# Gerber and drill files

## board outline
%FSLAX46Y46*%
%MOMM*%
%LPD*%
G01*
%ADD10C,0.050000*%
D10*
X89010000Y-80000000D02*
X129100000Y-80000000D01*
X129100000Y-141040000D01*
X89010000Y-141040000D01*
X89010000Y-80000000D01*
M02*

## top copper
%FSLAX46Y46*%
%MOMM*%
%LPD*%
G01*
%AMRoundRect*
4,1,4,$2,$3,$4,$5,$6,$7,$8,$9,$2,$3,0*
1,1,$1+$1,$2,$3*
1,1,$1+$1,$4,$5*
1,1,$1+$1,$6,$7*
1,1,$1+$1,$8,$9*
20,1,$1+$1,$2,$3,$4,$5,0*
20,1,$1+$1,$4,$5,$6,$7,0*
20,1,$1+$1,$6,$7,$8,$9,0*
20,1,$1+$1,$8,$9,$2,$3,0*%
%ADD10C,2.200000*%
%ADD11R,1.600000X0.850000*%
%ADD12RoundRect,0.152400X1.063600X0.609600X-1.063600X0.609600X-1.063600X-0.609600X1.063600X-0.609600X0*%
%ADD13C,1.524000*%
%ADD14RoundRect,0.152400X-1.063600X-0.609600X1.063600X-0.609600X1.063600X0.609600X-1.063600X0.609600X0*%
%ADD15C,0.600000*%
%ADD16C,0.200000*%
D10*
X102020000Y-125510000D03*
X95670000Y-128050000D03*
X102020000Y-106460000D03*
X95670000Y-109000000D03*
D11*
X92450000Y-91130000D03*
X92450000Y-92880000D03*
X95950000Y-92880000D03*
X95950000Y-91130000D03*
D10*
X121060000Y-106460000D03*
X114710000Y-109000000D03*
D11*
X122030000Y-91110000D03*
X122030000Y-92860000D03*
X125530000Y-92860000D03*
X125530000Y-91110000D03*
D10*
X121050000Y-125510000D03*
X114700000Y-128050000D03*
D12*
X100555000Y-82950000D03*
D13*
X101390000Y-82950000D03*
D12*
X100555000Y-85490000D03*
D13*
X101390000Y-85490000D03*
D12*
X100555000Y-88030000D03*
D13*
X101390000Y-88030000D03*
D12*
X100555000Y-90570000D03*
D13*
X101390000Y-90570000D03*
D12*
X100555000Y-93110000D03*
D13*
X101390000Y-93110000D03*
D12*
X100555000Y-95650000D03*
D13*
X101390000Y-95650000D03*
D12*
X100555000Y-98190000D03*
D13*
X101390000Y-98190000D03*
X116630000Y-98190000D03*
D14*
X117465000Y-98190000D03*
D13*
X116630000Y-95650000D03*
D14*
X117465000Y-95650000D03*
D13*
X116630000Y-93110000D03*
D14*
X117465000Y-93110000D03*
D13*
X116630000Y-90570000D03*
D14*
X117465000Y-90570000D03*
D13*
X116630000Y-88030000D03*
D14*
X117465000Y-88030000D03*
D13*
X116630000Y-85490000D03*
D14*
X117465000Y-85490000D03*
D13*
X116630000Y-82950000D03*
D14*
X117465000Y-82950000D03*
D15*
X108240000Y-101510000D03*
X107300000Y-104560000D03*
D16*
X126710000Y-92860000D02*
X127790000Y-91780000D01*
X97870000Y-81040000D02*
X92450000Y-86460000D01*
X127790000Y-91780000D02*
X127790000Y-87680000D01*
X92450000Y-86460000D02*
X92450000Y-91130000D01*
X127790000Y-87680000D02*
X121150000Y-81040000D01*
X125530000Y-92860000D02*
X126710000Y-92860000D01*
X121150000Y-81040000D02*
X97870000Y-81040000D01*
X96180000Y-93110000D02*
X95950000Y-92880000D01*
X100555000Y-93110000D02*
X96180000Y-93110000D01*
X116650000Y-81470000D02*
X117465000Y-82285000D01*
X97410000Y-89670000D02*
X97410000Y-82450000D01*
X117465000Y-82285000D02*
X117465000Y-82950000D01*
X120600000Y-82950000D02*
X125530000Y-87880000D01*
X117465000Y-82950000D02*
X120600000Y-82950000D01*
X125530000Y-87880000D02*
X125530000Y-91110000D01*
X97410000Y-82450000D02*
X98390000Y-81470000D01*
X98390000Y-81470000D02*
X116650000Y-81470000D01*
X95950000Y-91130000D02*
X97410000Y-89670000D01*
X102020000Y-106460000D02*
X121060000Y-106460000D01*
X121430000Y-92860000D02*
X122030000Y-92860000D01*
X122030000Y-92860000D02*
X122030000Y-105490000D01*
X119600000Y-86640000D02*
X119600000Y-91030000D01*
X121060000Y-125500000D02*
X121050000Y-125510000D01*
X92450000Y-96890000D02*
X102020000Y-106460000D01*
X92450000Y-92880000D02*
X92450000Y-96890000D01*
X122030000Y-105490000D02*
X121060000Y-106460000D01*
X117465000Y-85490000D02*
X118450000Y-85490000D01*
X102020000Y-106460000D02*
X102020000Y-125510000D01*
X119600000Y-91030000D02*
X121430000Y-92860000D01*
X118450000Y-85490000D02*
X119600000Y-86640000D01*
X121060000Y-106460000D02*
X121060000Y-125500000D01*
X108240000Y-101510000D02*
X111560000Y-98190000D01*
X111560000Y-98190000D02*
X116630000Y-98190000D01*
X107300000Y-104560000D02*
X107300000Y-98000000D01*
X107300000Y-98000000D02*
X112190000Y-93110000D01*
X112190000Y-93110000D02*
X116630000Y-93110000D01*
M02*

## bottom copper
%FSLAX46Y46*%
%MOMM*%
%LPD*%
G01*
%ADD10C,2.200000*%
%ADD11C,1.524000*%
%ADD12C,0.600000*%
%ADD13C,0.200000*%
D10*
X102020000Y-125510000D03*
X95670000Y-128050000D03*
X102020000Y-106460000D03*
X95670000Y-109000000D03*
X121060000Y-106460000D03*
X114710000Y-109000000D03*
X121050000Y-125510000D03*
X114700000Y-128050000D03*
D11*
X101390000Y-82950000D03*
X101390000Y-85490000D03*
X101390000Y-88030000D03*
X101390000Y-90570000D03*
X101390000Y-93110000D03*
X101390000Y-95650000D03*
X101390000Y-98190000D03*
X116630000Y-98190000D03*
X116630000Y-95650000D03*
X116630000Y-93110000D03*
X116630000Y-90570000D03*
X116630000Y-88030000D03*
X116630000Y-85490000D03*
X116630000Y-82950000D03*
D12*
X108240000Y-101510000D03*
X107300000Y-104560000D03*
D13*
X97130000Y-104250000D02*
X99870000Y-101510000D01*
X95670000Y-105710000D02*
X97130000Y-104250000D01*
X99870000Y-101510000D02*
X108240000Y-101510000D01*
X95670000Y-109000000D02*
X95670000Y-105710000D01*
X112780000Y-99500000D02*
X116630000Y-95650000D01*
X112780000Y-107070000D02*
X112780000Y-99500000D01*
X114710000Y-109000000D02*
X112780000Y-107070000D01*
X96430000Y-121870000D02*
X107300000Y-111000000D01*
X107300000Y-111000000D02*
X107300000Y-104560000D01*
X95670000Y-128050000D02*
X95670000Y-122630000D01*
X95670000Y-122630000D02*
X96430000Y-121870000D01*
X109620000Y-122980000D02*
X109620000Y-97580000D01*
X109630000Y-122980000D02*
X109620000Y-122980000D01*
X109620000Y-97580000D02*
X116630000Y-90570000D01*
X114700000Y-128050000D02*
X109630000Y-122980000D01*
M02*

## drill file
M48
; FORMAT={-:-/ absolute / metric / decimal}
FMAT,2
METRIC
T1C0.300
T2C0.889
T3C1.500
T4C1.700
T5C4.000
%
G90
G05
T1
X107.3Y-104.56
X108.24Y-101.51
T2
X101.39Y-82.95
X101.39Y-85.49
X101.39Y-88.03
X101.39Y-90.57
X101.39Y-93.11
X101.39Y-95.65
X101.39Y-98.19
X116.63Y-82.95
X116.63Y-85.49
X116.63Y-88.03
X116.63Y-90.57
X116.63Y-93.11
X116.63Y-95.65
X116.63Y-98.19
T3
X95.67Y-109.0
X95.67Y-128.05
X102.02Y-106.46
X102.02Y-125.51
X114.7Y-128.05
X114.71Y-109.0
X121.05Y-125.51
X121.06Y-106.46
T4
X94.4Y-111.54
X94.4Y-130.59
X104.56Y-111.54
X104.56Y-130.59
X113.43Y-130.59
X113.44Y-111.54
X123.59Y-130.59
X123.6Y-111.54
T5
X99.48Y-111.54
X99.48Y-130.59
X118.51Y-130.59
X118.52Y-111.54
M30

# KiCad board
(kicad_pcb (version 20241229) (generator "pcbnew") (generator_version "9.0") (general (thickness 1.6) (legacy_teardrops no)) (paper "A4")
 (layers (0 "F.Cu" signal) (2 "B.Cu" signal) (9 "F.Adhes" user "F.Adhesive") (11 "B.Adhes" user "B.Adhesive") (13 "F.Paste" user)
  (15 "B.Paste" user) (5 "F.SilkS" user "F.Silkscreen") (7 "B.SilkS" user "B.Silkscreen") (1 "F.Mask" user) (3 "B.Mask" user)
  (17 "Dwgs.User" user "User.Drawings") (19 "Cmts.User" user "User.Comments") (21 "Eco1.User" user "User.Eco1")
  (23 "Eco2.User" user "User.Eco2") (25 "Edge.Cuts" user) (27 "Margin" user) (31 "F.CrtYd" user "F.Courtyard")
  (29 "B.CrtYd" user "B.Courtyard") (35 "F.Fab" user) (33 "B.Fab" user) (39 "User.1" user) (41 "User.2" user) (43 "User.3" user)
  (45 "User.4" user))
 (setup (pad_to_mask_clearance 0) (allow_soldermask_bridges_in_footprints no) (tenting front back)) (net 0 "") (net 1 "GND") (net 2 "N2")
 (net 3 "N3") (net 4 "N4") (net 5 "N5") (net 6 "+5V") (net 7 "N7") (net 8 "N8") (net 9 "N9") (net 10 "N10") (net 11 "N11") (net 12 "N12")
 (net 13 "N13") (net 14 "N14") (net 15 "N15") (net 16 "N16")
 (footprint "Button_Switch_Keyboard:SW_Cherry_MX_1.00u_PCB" (layer "F.Cu") (at 102.02 125.51)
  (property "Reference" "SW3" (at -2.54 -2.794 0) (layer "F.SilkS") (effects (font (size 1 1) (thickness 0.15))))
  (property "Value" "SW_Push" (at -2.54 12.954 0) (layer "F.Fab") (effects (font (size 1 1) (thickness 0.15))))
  (pad "" np_thru_hole circle (at -7.62 5.08) (size 1.7 1.7) (drill 1.7) (layers "*.Cu" "*.Mask"))
  (pad "" np_thru_hole circle (at -2.54 5.08) (size 4 4) (drill 4) (layers "*.Cu" "*.Mask"))
  (pad "" np_thru_hole circle (at 2.54 5.08) (size 1.7 1.7) (drill 1.7) (layers "*.Cu" "*.Mask"))
  (pad "1" thru_hole circle (at 0 0) (size 2.2 2.2) (drill 1.5) (layers "*.Cu" "*.Mask") (remove_unused_layers no) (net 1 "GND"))
  (pad "2" thru_hole circle (at -6.35 2.54) (size 2.2 2.2) (drill 1.5) (layers "*.Cu" "*.Mask") (remove_unused_layers no) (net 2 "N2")))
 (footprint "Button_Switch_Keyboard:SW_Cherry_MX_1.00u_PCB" (layer "F.Cu") (at 102.02 106.46)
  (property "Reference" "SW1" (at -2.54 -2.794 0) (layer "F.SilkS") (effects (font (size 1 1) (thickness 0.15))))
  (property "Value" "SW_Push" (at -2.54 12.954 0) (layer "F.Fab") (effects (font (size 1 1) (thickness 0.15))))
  (pad "" np_thru_hole circle (at -7.62 5.08) (size 1.7 1.7) (drill 1.7) (layers "*.Cu" "*.Mask"))
  (pad "" np_thru_hole circle (at -2.54 5.08) (size 4 4) (drill 4) (layers "*.Cu" "*.Mask"))
  (pad "" np_thru_hole circle (at 2.54 5.08) (size 1.7 1.7) (drill 1.7) (layers "*.Cu" "*.Mask"))
  (pad "1" thru_hole circle (at 0 0) (size 2.2 2.2) (drill 1.5) (layers "*.Cu" "*.Mask") (remove_unused_layers no) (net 1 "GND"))
  (pad "2" thru_hole circle (at -6.35 2.54) (size 2.2 2.2) (drill 1.5) (layers "*.Cu" "*.Mask") (remove_unused_layers no) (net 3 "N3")))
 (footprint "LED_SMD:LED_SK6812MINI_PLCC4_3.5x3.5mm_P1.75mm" (layer "F.Cu") (at 94.2 92.005)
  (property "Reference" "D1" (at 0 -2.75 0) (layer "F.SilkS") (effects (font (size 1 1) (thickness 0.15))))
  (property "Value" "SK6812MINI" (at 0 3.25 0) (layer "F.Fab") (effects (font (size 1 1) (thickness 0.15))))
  (pad "1" smd rect (at -1.75 -0.875) (size 1.6 0.85) (layers "F.Cu" "F.Mask" "F.Paste") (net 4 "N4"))
  (pad "2" smd rect (at -1.75 0.875) (size 1.6 0.85) (layers "F.Cu" "F.Mask" "F.Paste") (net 1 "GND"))
  (pad "3" smd rect (at 1.75 0.875) (size 1.6 0.85) (layers "F.Cu" "F.Mask" "F.Paste") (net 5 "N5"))
  (pad "4" smd rect (at 1.75 -0.875) (size 1.6 0.85) (layers "F.Cu" "F.Mask" "F.Paste") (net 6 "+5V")))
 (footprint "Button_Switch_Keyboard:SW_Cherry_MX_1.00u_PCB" (layer "F.Cu") (at 121.06 106.46)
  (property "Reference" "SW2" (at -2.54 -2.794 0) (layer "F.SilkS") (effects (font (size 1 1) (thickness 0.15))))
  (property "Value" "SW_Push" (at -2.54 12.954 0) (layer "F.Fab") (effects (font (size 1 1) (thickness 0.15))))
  (pad "" np_thru_hole circle (at -7.62 5.08) (size 1.7 1.7) (drill 1.7) (layers "*.Cu" "*.Mask"))
  (pad "" np_thru_hole circle (at -2.54 5.08) (size 4 4) (drill 4) (layers "*.Cu" "*.Mask"))
  (pad "" np_thru_hole circle (at 2.54 5.08) (size 1.7 1.7) (drill 1.7) (layers "*.Cu" "*.Mask"))
  (pad "1" thru_hole circle (at 0 0) (size 2.2 2.2) (drill 1.5) (layers "*.Cu" "*.Mask") (remove_unused_layers no) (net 1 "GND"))
  (pad "2" thru_hole circle (at -6.35 2.54) (size 2.2 2.2) (drill 1.5) (layers "*.Cu" "*.Mask") (remove_unused_layers no) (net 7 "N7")))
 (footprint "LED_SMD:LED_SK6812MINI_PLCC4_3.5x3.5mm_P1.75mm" (layer "F.Cu") (at 123.78 91.985)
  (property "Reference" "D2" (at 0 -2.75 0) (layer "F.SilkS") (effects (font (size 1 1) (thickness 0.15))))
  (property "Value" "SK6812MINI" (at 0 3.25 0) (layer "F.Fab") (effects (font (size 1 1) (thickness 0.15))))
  (pad "1" smd rect (at -1.75 -0.875) (size 1.6 0.85) (layers "F.Cu" "F.Mask" "F.Paste") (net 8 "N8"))
  (pad "2" smd rect (at -1.75 0.875) (size 1.6 0.85) (layers "F.Cu" "F.Mask" "F.Paste") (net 1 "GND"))
  (pad "3" smd rect (at 1.75 0.875) (size 1.6 0.85) (layers "F.Cu" "F.Mask" "F.Paste") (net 4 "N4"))
  (pad "4" smd rect (at 1.75 -0.875) (size 1.6 0.85) (layers "F.Cu" "F.Mask" "F.Paste") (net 6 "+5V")))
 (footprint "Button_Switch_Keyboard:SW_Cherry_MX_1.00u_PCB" (layer "F.Cu") (at 121.05 125.51)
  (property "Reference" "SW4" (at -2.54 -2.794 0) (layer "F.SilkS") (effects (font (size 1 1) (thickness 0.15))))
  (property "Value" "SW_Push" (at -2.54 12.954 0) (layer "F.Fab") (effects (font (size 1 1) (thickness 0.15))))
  (pad "" np_thru_hole circle (at -7.62 5.08) (size 1.7 1.7) (drill 1.7) (layers "*.Cu" "*.Mask"))
  (pad "" np_thru_hole circle (at -2.54 5.08) (size 4 4) (drill 4) (layers "*.Cu" "*.Mask"))
  (pad "" np_thru_hole circle (at 2.54 5.08) (size 1.7 1.7) (drill 1.7) (layers "*.Cu" "*.Mask"))
  (pad "1" thru_hole circle (at 0 0) (size 2.2 2.2) (drill 1.5) (layers "*.Cu" "*.Mask") (remove_unused_layers no) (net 1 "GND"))
  (pad "2" thru_hole circle (at -6.35 2.54) (size 2.2 2.2) (drill 1.5) (layers "*.Cu" "*.Mask") (remove_unused_layers no) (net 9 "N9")))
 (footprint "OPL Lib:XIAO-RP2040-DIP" (layer "F.Cu") (at 109.01 90.57)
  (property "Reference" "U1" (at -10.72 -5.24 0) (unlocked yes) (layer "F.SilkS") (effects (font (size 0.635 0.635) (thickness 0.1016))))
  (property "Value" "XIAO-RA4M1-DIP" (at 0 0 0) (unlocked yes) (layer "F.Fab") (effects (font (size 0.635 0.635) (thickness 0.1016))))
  (pad "1" smd roundrect (at -8.455 -7.62 180) (size 2.432 1.524) (layers "F.Cu" "F.Mask") (roundrect_rratio 0.1) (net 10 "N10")
   (thermal_bridge_angle 45))
  (pad "1" thru_hole circle (at -7.62 -7.62 180) (size 1.524 1.524) (drill 0.889) (layers "*.Cu" "*.Mask") (remove_unused_layers no)
   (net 10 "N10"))
  (pad "2" smd roundrect (at -8.455 -5.08 180) (size 2.432 1.524) (layers "F.Cu" "F.Mask") (roundrect_rratio 0.1) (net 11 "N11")
   (thermal_bridge_angle 45))
  (pad "2" thru_hole circle (at -7.62 -5.08 180) (size 1.524 1.524) (drill 0.889) (layers "*.Cu" "*.Mask") (remove_unused_layers no)
   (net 11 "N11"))
  (pad "3" smd roundrect (at -8.455 -2.54 180) (size 2.432 1.524) (layers "F.Cu" "F.Mask") (roundrect_rratio 0.1) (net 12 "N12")
   (thermal_bridge_angle 45))
  (pad "3" thru_hole circle (at -7.62 -2.54 180) (size 1.524 1.524) (drill 0.889) (layers "*.Cu" "*.Mask") (remove_unused_layers no)
   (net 12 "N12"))
  (pad "4" smd roundrect (at -8.455 0 180) (size 2.432 1.524) (layers "F.Cu" "F.Mask") (roundrect_rratio 0.1) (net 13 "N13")
   (thermal_bridge_angle 45))
  (pad "4" thru_hole circle (at -7.62 0 180) (size 1.524 1.524) (drill 0.889) (layers "*.Cu" "*.Mask") (remove_unused_layers no)
   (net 13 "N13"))
  (pad "5" smd roundrect (at -8.455 2.54 180) (size 2.432 1.524) (layers "F.Cu" "F.Mask") (roundrect_rratio 0.1) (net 5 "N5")
   (thermal_bridge_angle 45))
  (pad "5" thru_hole circle (at -7.62 2.54 180) (size 1.524 1.524) (drill 0.889) (layers "*.Cu" "*.Mask") (remove_unused_layers no)
   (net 5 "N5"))
  (pad "6" smd roundrect (at -8.455 5.08 180) (size 2.432 1.524) (layers "F.Cu" "F.Mask") (roundrect_rratio 0.1) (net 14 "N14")
   (thermal_bridge_angle 45))
  (pad "6" thru_hole circle (at -7.62 5.08 180) (size 1.524 1.524) (drill 0.889) (layers "*.Cu" "*.Mask") (remove_unused_layers no)
   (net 14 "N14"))
  (pad "7" smd roundrect (at -8.455 7.62 180) (size 2.432 1.524) (layers "F.Cu" "F.Mask") (roundrect_rratio 0.1) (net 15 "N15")
   (thermal_bridge_angle 45))
  (pad "7" thru_hole circle (at -7.62 7.62 180) (size 1.524 1.524) (drill 0.889) (layers "*.Cu" "*.Mask") (remove_unused_layers no)
   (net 15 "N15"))
  (pad "8" thru_hole circle (at 7.62 7.62) (size 1.524 1.524) (drill 0.889) (layers "*.Cu" "*.Mask") (remove_unused_layers no) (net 3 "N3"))
  (pad "8" smd roundrect (at 8.455 7.62) (size 2.432 1.524) (layers "F.Cu" "F.Mask") (roundrect_rratio 0.1) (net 3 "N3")
   (thermal_bridge_angle 45))
  (pad "9" thru_hole circle (at 7.62 5.08) (size 1.524 1.524) (drill 0.889) (layers "*.Cu" "*.Mask") (remove_unused_layers no) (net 7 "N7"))
  (pad "9" smd roundrect (at 8.455 5.08) (size 2.432 1.524) (layers "F.Cu" "F.Mask") (roundrect_rratio 0.1) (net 7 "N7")
   (thermal_bridge_angle 45))
  (pad "10" thru_hole circle (at 7.62 2.54) (size 1.524 1.524) (drill 0.889) (layers "*.Cu" "*.Mask") (remove_unused_layers no) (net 2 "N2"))
  (pad "10" smd roundrect (at 8.455 2.54) (size 2.432 1.524) (layers "F.Cu" "F.Mask") (roundrect_rratio 0.1) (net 2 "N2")
   (thermal_bridge_angle 45))
  (pad "11" thru_hole circle (at 7.62 0) (size 1.524 1.524) (drill 0.889) (layers "*.Cu" "*.Mask") (remove_unused_layers no) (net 9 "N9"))
  (pad "11" smd roundrect (at 8.455 0) (size 2.432 1.524) (layers "F.Cu" "F.Mask") (roundrect_rratio 0.1) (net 9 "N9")
   (thermal_bridge_angle 45))
  (pad "12" thru_hole circle (at 7.62 -2.54) (size 1.524 1.524) (drill 0.889) (layers "*.Cu" "*.Mask") (remove_unused_layers no)
   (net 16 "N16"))
  (pad "12" smd roundrect (at 8.455 -2.54) (size 2.432 1.524) (layers "F.Cu" "F.Mask") (roundrect_rratio 0.1) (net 16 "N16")
   (thermal_bridge_angle 45))
  (pad "13" thru_hole circle (at 7.62 -5.08) (size 1.524 1.524) (drill 0.889) (layers "*.Cu" "*.Mask") (remove_unused_layers no)
   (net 1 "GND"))
  (pad "13" smd roundrect (at 8.455 -5.08) (size 2.432 1.524) (layers "F.Cu" "F.Mask") (roundrect_rratio 0.1) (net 1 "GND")
   (thermal_bridge_angle 45))
  (pad "14" thru_hole circle (at 7.62 -7.62) (size 1.524 1.524) (drill 0.889) (layers "*.Cu" "*.Mask") (remove_unused_layers no)
   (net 6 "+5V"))
  (pad "14" smd roundrect (at 8.455 -7.62) (size 2.432 1.524) (layers "F.Cu" "F.Mask") (roundrect_rratio 0.1) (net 6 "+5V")
   (thermal_bridge_angle 45)))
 (gr_rect (start 89.01 80) (end 129.1 141.04) (stroke (width 0.05) (type default)) (fill no) (layer "Edge.Cuts"))
 (segment (start 126.71 92.86) (end 127.79 91.78) (width 0.2) (layer "F.Cu") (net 4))
 (segment (start 97.87 81.04) (end 92.45 86.46) (width 0.2) (layer "F.Cu") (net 4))
 (segment (start 127.79 91.78) (end 127.79 87.68) (width 0.2) (layer "F.Cu") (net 4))
 (segment (start 92.45 86.46) (end 92.45 91.13) (width 0.2) (layer "F.Cu") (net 4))
 (segment (start 127.79 87.68) (end 121.15 81.04) (width 0.2) (layer "F.Cu") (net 4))
 (segment (start 125.53 92.86) (end 126.71 92.86) (width 0.2) (layer "F.Cu") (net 4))
 (segment (start 121.15 81.04) (end 97.87 81.04) (width 0.2) (layer "F.Cu") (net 4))
 (segment (start 96.18 93.11) (end 95.95 92.88) (width 0.2) (layer "F.Cu") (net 5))
 (segment (start 100.555 93.11) (end 96.18 93.11) (width 0.2) (layer "F.Cu") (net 5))
 (segment (start 116.65 81.47) (end 117.465 82.285) (width 0.2) (layer "F.Cu") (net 6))
 (segment (start 97.41 89.67) (end 97.41 82.45) (width 0.2) (layer "F.Cu") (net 6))
 (segment (start 117.465 82.285) (end 117.465 82.95) (width 0.2) (layer "F.Cu") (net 6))
 (segment (start 120.6 82.95) (end 125.53 87.88) (width 0.2) (layer "F.Cu") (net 6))
 (segment (start 117.465 82.95) (end 120.6 82.95) (width 0.2) (layer "F.Cu") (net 6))
 (segment (start 125.53 87.88) (end 125.53 91.11) (width 0.2) (layer "F.Cu") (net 6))
 (segment (start 97.41 82.45) (end 98.39 81.47) (width 0.2) (layer "F.Cu") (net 6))
 (segment (start 98.39 81.47) (end 116.65 81.47) (width 0.2) (layer "F.Cu") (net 6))
 (segment (start 95.95 91.13) (end 97.41 89.67) (width 0.2) (layer "F.Cu") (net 6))
 (segment (start 102.02 106.46) (end 121.06 106.46) (width 0.2) (layer "F.Cu") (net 1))
 (segment (start 121.43 92.86) (end 122.03 92.86) (width 0.2) (layer "F.Cu") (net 1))
 (segment (start 122.03 92.86) (end 122.03 105.49) (width 0.2) (layer "F.Cu") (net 1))
 (segment (start 119.6 86.64) (end 119.6 91.03) (width 0.2) (layer "F.Cu") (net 1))
 (segment (start 121.06 125.5) (end 121.05 125.51) (width 0.2) (layer "F.Cu") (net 1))
 (segment (start 92.45 96.89) (end 102.02 106.46) (width 0.2) (layer "F.Cu") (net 1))
 (segment (start 92.45 92.88) (end 92.45 96.89) (width 0.2) (layer "F.Cu") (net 1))
 (segment (start 122.03 105.49) (end 121.06 106.46) (width 0.2) (layer "F.Cu") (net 1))
 (segment (start 117.465 85.49) (end 118.45 85.49) (width 0.2) (layer "F.Cu") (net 1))
 (segment (start 102.02 106.46) (end 102.02 125.51) (width 0.2) (layer "F.Cu") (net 1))
 (segment (start 119.6 91.03) (end 121.43 92.86) (width 0.2) (layer "F.Cu") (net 1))
 (segment (start 118.45 85.49) (end 119.6 86.64) (width 0.2) (layer "F.Cu") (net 1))
 (segment (start 121.06 106.46) (end 121.06 125.5) (width 0.2) (layer "F.Cu") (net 1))
 (segment (start 108.24 101.51) (end 111.56 98.19) (width 0.2) (layer "F.Cu") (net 3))
 (segment (start 111.56 98.19) (end 116.63 98.19) (width 0.2) (layer "F.Cu") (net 3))
 (via (at 108.24 101.51) (size 0.6) (drill 0.3) (layers "F.Cu" "B.Cu") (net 3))
 (segment (start 97.13 104.25) (end 99.87 101.51) (width 0.2) (layer "B.Cu") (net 3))
 (segment (start 95.67 105.71) (end 97.13 104.25) (width 0.2) (layer "B.Cu") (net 3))
 (segment (start 99.87 101.51) (end 108.24 101.51) (width 0.2) (layer "B.Cu") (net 3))
 (segment (start 95.67 109) (end 95.67 105.71) (width 0.2) (layer "B.Cu") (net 3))
 (segment (start 112.78 99.5) (end 116.63 95.65) (width 0.2) (layer "B.Cu") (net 7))
 (segment (start 112.78 107.07) (end 112.78 99.5) (width 0.2) (layer "B.Cu") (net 7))
 (segment (start 114.71 109) (end 112.78 107.07) (width 0.2) (layer "B.Cu") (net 7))
 (segment (start 107.3 104.56) (end 107.3 98) (width 0.2) (layer "F.Cu") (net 2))
 (segment (start 107.3 98) (end 112.19 93.11) (width 0.2) (layer "F.Cu") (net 2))
 (segment (start 112.19 93.11) (end 116.63 93.11) (width 0.2) (layer "F.Cu") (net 2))
 (via (at 107.3 104.56) (size 0.6) (drill 0.3) (layers "F.Cu" "B.Cu") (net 2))
 (segment (start 96.43 121.87) (end 107.3 111) (width 0.2) (layer "B.Cu") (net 2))
 (segment (start 107.3 111) (end 107.3 104.56) (width 0.2) (layer "B.Cu") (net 2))
 (segment (start 95.67 128.05) (end 95.67 122.63) (width 0.2) (layer "B.Cu") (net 2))
 (segment (start 95.67 122.63) (end 96.43 121.87) (width 0.2) (layer "B.Cu") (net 2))
 (segment (start 109.62 122.98) (end 109.62 97.58) (width 0.2) (layer "B.Cu") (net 9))
 (segment (start 109.63 122.98) (end 109.62 122.98) (width 0.2) (layer "B.Cu") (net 9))
 (segment (start 109.62 97.58) (end 116.63 90.57) (width 0.2) (layer "B.Cu") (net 9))
 (segment (start 114.7 128.05) (end 109.63 122.98) (width 0.2) (layer "B.Cu") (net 9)))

